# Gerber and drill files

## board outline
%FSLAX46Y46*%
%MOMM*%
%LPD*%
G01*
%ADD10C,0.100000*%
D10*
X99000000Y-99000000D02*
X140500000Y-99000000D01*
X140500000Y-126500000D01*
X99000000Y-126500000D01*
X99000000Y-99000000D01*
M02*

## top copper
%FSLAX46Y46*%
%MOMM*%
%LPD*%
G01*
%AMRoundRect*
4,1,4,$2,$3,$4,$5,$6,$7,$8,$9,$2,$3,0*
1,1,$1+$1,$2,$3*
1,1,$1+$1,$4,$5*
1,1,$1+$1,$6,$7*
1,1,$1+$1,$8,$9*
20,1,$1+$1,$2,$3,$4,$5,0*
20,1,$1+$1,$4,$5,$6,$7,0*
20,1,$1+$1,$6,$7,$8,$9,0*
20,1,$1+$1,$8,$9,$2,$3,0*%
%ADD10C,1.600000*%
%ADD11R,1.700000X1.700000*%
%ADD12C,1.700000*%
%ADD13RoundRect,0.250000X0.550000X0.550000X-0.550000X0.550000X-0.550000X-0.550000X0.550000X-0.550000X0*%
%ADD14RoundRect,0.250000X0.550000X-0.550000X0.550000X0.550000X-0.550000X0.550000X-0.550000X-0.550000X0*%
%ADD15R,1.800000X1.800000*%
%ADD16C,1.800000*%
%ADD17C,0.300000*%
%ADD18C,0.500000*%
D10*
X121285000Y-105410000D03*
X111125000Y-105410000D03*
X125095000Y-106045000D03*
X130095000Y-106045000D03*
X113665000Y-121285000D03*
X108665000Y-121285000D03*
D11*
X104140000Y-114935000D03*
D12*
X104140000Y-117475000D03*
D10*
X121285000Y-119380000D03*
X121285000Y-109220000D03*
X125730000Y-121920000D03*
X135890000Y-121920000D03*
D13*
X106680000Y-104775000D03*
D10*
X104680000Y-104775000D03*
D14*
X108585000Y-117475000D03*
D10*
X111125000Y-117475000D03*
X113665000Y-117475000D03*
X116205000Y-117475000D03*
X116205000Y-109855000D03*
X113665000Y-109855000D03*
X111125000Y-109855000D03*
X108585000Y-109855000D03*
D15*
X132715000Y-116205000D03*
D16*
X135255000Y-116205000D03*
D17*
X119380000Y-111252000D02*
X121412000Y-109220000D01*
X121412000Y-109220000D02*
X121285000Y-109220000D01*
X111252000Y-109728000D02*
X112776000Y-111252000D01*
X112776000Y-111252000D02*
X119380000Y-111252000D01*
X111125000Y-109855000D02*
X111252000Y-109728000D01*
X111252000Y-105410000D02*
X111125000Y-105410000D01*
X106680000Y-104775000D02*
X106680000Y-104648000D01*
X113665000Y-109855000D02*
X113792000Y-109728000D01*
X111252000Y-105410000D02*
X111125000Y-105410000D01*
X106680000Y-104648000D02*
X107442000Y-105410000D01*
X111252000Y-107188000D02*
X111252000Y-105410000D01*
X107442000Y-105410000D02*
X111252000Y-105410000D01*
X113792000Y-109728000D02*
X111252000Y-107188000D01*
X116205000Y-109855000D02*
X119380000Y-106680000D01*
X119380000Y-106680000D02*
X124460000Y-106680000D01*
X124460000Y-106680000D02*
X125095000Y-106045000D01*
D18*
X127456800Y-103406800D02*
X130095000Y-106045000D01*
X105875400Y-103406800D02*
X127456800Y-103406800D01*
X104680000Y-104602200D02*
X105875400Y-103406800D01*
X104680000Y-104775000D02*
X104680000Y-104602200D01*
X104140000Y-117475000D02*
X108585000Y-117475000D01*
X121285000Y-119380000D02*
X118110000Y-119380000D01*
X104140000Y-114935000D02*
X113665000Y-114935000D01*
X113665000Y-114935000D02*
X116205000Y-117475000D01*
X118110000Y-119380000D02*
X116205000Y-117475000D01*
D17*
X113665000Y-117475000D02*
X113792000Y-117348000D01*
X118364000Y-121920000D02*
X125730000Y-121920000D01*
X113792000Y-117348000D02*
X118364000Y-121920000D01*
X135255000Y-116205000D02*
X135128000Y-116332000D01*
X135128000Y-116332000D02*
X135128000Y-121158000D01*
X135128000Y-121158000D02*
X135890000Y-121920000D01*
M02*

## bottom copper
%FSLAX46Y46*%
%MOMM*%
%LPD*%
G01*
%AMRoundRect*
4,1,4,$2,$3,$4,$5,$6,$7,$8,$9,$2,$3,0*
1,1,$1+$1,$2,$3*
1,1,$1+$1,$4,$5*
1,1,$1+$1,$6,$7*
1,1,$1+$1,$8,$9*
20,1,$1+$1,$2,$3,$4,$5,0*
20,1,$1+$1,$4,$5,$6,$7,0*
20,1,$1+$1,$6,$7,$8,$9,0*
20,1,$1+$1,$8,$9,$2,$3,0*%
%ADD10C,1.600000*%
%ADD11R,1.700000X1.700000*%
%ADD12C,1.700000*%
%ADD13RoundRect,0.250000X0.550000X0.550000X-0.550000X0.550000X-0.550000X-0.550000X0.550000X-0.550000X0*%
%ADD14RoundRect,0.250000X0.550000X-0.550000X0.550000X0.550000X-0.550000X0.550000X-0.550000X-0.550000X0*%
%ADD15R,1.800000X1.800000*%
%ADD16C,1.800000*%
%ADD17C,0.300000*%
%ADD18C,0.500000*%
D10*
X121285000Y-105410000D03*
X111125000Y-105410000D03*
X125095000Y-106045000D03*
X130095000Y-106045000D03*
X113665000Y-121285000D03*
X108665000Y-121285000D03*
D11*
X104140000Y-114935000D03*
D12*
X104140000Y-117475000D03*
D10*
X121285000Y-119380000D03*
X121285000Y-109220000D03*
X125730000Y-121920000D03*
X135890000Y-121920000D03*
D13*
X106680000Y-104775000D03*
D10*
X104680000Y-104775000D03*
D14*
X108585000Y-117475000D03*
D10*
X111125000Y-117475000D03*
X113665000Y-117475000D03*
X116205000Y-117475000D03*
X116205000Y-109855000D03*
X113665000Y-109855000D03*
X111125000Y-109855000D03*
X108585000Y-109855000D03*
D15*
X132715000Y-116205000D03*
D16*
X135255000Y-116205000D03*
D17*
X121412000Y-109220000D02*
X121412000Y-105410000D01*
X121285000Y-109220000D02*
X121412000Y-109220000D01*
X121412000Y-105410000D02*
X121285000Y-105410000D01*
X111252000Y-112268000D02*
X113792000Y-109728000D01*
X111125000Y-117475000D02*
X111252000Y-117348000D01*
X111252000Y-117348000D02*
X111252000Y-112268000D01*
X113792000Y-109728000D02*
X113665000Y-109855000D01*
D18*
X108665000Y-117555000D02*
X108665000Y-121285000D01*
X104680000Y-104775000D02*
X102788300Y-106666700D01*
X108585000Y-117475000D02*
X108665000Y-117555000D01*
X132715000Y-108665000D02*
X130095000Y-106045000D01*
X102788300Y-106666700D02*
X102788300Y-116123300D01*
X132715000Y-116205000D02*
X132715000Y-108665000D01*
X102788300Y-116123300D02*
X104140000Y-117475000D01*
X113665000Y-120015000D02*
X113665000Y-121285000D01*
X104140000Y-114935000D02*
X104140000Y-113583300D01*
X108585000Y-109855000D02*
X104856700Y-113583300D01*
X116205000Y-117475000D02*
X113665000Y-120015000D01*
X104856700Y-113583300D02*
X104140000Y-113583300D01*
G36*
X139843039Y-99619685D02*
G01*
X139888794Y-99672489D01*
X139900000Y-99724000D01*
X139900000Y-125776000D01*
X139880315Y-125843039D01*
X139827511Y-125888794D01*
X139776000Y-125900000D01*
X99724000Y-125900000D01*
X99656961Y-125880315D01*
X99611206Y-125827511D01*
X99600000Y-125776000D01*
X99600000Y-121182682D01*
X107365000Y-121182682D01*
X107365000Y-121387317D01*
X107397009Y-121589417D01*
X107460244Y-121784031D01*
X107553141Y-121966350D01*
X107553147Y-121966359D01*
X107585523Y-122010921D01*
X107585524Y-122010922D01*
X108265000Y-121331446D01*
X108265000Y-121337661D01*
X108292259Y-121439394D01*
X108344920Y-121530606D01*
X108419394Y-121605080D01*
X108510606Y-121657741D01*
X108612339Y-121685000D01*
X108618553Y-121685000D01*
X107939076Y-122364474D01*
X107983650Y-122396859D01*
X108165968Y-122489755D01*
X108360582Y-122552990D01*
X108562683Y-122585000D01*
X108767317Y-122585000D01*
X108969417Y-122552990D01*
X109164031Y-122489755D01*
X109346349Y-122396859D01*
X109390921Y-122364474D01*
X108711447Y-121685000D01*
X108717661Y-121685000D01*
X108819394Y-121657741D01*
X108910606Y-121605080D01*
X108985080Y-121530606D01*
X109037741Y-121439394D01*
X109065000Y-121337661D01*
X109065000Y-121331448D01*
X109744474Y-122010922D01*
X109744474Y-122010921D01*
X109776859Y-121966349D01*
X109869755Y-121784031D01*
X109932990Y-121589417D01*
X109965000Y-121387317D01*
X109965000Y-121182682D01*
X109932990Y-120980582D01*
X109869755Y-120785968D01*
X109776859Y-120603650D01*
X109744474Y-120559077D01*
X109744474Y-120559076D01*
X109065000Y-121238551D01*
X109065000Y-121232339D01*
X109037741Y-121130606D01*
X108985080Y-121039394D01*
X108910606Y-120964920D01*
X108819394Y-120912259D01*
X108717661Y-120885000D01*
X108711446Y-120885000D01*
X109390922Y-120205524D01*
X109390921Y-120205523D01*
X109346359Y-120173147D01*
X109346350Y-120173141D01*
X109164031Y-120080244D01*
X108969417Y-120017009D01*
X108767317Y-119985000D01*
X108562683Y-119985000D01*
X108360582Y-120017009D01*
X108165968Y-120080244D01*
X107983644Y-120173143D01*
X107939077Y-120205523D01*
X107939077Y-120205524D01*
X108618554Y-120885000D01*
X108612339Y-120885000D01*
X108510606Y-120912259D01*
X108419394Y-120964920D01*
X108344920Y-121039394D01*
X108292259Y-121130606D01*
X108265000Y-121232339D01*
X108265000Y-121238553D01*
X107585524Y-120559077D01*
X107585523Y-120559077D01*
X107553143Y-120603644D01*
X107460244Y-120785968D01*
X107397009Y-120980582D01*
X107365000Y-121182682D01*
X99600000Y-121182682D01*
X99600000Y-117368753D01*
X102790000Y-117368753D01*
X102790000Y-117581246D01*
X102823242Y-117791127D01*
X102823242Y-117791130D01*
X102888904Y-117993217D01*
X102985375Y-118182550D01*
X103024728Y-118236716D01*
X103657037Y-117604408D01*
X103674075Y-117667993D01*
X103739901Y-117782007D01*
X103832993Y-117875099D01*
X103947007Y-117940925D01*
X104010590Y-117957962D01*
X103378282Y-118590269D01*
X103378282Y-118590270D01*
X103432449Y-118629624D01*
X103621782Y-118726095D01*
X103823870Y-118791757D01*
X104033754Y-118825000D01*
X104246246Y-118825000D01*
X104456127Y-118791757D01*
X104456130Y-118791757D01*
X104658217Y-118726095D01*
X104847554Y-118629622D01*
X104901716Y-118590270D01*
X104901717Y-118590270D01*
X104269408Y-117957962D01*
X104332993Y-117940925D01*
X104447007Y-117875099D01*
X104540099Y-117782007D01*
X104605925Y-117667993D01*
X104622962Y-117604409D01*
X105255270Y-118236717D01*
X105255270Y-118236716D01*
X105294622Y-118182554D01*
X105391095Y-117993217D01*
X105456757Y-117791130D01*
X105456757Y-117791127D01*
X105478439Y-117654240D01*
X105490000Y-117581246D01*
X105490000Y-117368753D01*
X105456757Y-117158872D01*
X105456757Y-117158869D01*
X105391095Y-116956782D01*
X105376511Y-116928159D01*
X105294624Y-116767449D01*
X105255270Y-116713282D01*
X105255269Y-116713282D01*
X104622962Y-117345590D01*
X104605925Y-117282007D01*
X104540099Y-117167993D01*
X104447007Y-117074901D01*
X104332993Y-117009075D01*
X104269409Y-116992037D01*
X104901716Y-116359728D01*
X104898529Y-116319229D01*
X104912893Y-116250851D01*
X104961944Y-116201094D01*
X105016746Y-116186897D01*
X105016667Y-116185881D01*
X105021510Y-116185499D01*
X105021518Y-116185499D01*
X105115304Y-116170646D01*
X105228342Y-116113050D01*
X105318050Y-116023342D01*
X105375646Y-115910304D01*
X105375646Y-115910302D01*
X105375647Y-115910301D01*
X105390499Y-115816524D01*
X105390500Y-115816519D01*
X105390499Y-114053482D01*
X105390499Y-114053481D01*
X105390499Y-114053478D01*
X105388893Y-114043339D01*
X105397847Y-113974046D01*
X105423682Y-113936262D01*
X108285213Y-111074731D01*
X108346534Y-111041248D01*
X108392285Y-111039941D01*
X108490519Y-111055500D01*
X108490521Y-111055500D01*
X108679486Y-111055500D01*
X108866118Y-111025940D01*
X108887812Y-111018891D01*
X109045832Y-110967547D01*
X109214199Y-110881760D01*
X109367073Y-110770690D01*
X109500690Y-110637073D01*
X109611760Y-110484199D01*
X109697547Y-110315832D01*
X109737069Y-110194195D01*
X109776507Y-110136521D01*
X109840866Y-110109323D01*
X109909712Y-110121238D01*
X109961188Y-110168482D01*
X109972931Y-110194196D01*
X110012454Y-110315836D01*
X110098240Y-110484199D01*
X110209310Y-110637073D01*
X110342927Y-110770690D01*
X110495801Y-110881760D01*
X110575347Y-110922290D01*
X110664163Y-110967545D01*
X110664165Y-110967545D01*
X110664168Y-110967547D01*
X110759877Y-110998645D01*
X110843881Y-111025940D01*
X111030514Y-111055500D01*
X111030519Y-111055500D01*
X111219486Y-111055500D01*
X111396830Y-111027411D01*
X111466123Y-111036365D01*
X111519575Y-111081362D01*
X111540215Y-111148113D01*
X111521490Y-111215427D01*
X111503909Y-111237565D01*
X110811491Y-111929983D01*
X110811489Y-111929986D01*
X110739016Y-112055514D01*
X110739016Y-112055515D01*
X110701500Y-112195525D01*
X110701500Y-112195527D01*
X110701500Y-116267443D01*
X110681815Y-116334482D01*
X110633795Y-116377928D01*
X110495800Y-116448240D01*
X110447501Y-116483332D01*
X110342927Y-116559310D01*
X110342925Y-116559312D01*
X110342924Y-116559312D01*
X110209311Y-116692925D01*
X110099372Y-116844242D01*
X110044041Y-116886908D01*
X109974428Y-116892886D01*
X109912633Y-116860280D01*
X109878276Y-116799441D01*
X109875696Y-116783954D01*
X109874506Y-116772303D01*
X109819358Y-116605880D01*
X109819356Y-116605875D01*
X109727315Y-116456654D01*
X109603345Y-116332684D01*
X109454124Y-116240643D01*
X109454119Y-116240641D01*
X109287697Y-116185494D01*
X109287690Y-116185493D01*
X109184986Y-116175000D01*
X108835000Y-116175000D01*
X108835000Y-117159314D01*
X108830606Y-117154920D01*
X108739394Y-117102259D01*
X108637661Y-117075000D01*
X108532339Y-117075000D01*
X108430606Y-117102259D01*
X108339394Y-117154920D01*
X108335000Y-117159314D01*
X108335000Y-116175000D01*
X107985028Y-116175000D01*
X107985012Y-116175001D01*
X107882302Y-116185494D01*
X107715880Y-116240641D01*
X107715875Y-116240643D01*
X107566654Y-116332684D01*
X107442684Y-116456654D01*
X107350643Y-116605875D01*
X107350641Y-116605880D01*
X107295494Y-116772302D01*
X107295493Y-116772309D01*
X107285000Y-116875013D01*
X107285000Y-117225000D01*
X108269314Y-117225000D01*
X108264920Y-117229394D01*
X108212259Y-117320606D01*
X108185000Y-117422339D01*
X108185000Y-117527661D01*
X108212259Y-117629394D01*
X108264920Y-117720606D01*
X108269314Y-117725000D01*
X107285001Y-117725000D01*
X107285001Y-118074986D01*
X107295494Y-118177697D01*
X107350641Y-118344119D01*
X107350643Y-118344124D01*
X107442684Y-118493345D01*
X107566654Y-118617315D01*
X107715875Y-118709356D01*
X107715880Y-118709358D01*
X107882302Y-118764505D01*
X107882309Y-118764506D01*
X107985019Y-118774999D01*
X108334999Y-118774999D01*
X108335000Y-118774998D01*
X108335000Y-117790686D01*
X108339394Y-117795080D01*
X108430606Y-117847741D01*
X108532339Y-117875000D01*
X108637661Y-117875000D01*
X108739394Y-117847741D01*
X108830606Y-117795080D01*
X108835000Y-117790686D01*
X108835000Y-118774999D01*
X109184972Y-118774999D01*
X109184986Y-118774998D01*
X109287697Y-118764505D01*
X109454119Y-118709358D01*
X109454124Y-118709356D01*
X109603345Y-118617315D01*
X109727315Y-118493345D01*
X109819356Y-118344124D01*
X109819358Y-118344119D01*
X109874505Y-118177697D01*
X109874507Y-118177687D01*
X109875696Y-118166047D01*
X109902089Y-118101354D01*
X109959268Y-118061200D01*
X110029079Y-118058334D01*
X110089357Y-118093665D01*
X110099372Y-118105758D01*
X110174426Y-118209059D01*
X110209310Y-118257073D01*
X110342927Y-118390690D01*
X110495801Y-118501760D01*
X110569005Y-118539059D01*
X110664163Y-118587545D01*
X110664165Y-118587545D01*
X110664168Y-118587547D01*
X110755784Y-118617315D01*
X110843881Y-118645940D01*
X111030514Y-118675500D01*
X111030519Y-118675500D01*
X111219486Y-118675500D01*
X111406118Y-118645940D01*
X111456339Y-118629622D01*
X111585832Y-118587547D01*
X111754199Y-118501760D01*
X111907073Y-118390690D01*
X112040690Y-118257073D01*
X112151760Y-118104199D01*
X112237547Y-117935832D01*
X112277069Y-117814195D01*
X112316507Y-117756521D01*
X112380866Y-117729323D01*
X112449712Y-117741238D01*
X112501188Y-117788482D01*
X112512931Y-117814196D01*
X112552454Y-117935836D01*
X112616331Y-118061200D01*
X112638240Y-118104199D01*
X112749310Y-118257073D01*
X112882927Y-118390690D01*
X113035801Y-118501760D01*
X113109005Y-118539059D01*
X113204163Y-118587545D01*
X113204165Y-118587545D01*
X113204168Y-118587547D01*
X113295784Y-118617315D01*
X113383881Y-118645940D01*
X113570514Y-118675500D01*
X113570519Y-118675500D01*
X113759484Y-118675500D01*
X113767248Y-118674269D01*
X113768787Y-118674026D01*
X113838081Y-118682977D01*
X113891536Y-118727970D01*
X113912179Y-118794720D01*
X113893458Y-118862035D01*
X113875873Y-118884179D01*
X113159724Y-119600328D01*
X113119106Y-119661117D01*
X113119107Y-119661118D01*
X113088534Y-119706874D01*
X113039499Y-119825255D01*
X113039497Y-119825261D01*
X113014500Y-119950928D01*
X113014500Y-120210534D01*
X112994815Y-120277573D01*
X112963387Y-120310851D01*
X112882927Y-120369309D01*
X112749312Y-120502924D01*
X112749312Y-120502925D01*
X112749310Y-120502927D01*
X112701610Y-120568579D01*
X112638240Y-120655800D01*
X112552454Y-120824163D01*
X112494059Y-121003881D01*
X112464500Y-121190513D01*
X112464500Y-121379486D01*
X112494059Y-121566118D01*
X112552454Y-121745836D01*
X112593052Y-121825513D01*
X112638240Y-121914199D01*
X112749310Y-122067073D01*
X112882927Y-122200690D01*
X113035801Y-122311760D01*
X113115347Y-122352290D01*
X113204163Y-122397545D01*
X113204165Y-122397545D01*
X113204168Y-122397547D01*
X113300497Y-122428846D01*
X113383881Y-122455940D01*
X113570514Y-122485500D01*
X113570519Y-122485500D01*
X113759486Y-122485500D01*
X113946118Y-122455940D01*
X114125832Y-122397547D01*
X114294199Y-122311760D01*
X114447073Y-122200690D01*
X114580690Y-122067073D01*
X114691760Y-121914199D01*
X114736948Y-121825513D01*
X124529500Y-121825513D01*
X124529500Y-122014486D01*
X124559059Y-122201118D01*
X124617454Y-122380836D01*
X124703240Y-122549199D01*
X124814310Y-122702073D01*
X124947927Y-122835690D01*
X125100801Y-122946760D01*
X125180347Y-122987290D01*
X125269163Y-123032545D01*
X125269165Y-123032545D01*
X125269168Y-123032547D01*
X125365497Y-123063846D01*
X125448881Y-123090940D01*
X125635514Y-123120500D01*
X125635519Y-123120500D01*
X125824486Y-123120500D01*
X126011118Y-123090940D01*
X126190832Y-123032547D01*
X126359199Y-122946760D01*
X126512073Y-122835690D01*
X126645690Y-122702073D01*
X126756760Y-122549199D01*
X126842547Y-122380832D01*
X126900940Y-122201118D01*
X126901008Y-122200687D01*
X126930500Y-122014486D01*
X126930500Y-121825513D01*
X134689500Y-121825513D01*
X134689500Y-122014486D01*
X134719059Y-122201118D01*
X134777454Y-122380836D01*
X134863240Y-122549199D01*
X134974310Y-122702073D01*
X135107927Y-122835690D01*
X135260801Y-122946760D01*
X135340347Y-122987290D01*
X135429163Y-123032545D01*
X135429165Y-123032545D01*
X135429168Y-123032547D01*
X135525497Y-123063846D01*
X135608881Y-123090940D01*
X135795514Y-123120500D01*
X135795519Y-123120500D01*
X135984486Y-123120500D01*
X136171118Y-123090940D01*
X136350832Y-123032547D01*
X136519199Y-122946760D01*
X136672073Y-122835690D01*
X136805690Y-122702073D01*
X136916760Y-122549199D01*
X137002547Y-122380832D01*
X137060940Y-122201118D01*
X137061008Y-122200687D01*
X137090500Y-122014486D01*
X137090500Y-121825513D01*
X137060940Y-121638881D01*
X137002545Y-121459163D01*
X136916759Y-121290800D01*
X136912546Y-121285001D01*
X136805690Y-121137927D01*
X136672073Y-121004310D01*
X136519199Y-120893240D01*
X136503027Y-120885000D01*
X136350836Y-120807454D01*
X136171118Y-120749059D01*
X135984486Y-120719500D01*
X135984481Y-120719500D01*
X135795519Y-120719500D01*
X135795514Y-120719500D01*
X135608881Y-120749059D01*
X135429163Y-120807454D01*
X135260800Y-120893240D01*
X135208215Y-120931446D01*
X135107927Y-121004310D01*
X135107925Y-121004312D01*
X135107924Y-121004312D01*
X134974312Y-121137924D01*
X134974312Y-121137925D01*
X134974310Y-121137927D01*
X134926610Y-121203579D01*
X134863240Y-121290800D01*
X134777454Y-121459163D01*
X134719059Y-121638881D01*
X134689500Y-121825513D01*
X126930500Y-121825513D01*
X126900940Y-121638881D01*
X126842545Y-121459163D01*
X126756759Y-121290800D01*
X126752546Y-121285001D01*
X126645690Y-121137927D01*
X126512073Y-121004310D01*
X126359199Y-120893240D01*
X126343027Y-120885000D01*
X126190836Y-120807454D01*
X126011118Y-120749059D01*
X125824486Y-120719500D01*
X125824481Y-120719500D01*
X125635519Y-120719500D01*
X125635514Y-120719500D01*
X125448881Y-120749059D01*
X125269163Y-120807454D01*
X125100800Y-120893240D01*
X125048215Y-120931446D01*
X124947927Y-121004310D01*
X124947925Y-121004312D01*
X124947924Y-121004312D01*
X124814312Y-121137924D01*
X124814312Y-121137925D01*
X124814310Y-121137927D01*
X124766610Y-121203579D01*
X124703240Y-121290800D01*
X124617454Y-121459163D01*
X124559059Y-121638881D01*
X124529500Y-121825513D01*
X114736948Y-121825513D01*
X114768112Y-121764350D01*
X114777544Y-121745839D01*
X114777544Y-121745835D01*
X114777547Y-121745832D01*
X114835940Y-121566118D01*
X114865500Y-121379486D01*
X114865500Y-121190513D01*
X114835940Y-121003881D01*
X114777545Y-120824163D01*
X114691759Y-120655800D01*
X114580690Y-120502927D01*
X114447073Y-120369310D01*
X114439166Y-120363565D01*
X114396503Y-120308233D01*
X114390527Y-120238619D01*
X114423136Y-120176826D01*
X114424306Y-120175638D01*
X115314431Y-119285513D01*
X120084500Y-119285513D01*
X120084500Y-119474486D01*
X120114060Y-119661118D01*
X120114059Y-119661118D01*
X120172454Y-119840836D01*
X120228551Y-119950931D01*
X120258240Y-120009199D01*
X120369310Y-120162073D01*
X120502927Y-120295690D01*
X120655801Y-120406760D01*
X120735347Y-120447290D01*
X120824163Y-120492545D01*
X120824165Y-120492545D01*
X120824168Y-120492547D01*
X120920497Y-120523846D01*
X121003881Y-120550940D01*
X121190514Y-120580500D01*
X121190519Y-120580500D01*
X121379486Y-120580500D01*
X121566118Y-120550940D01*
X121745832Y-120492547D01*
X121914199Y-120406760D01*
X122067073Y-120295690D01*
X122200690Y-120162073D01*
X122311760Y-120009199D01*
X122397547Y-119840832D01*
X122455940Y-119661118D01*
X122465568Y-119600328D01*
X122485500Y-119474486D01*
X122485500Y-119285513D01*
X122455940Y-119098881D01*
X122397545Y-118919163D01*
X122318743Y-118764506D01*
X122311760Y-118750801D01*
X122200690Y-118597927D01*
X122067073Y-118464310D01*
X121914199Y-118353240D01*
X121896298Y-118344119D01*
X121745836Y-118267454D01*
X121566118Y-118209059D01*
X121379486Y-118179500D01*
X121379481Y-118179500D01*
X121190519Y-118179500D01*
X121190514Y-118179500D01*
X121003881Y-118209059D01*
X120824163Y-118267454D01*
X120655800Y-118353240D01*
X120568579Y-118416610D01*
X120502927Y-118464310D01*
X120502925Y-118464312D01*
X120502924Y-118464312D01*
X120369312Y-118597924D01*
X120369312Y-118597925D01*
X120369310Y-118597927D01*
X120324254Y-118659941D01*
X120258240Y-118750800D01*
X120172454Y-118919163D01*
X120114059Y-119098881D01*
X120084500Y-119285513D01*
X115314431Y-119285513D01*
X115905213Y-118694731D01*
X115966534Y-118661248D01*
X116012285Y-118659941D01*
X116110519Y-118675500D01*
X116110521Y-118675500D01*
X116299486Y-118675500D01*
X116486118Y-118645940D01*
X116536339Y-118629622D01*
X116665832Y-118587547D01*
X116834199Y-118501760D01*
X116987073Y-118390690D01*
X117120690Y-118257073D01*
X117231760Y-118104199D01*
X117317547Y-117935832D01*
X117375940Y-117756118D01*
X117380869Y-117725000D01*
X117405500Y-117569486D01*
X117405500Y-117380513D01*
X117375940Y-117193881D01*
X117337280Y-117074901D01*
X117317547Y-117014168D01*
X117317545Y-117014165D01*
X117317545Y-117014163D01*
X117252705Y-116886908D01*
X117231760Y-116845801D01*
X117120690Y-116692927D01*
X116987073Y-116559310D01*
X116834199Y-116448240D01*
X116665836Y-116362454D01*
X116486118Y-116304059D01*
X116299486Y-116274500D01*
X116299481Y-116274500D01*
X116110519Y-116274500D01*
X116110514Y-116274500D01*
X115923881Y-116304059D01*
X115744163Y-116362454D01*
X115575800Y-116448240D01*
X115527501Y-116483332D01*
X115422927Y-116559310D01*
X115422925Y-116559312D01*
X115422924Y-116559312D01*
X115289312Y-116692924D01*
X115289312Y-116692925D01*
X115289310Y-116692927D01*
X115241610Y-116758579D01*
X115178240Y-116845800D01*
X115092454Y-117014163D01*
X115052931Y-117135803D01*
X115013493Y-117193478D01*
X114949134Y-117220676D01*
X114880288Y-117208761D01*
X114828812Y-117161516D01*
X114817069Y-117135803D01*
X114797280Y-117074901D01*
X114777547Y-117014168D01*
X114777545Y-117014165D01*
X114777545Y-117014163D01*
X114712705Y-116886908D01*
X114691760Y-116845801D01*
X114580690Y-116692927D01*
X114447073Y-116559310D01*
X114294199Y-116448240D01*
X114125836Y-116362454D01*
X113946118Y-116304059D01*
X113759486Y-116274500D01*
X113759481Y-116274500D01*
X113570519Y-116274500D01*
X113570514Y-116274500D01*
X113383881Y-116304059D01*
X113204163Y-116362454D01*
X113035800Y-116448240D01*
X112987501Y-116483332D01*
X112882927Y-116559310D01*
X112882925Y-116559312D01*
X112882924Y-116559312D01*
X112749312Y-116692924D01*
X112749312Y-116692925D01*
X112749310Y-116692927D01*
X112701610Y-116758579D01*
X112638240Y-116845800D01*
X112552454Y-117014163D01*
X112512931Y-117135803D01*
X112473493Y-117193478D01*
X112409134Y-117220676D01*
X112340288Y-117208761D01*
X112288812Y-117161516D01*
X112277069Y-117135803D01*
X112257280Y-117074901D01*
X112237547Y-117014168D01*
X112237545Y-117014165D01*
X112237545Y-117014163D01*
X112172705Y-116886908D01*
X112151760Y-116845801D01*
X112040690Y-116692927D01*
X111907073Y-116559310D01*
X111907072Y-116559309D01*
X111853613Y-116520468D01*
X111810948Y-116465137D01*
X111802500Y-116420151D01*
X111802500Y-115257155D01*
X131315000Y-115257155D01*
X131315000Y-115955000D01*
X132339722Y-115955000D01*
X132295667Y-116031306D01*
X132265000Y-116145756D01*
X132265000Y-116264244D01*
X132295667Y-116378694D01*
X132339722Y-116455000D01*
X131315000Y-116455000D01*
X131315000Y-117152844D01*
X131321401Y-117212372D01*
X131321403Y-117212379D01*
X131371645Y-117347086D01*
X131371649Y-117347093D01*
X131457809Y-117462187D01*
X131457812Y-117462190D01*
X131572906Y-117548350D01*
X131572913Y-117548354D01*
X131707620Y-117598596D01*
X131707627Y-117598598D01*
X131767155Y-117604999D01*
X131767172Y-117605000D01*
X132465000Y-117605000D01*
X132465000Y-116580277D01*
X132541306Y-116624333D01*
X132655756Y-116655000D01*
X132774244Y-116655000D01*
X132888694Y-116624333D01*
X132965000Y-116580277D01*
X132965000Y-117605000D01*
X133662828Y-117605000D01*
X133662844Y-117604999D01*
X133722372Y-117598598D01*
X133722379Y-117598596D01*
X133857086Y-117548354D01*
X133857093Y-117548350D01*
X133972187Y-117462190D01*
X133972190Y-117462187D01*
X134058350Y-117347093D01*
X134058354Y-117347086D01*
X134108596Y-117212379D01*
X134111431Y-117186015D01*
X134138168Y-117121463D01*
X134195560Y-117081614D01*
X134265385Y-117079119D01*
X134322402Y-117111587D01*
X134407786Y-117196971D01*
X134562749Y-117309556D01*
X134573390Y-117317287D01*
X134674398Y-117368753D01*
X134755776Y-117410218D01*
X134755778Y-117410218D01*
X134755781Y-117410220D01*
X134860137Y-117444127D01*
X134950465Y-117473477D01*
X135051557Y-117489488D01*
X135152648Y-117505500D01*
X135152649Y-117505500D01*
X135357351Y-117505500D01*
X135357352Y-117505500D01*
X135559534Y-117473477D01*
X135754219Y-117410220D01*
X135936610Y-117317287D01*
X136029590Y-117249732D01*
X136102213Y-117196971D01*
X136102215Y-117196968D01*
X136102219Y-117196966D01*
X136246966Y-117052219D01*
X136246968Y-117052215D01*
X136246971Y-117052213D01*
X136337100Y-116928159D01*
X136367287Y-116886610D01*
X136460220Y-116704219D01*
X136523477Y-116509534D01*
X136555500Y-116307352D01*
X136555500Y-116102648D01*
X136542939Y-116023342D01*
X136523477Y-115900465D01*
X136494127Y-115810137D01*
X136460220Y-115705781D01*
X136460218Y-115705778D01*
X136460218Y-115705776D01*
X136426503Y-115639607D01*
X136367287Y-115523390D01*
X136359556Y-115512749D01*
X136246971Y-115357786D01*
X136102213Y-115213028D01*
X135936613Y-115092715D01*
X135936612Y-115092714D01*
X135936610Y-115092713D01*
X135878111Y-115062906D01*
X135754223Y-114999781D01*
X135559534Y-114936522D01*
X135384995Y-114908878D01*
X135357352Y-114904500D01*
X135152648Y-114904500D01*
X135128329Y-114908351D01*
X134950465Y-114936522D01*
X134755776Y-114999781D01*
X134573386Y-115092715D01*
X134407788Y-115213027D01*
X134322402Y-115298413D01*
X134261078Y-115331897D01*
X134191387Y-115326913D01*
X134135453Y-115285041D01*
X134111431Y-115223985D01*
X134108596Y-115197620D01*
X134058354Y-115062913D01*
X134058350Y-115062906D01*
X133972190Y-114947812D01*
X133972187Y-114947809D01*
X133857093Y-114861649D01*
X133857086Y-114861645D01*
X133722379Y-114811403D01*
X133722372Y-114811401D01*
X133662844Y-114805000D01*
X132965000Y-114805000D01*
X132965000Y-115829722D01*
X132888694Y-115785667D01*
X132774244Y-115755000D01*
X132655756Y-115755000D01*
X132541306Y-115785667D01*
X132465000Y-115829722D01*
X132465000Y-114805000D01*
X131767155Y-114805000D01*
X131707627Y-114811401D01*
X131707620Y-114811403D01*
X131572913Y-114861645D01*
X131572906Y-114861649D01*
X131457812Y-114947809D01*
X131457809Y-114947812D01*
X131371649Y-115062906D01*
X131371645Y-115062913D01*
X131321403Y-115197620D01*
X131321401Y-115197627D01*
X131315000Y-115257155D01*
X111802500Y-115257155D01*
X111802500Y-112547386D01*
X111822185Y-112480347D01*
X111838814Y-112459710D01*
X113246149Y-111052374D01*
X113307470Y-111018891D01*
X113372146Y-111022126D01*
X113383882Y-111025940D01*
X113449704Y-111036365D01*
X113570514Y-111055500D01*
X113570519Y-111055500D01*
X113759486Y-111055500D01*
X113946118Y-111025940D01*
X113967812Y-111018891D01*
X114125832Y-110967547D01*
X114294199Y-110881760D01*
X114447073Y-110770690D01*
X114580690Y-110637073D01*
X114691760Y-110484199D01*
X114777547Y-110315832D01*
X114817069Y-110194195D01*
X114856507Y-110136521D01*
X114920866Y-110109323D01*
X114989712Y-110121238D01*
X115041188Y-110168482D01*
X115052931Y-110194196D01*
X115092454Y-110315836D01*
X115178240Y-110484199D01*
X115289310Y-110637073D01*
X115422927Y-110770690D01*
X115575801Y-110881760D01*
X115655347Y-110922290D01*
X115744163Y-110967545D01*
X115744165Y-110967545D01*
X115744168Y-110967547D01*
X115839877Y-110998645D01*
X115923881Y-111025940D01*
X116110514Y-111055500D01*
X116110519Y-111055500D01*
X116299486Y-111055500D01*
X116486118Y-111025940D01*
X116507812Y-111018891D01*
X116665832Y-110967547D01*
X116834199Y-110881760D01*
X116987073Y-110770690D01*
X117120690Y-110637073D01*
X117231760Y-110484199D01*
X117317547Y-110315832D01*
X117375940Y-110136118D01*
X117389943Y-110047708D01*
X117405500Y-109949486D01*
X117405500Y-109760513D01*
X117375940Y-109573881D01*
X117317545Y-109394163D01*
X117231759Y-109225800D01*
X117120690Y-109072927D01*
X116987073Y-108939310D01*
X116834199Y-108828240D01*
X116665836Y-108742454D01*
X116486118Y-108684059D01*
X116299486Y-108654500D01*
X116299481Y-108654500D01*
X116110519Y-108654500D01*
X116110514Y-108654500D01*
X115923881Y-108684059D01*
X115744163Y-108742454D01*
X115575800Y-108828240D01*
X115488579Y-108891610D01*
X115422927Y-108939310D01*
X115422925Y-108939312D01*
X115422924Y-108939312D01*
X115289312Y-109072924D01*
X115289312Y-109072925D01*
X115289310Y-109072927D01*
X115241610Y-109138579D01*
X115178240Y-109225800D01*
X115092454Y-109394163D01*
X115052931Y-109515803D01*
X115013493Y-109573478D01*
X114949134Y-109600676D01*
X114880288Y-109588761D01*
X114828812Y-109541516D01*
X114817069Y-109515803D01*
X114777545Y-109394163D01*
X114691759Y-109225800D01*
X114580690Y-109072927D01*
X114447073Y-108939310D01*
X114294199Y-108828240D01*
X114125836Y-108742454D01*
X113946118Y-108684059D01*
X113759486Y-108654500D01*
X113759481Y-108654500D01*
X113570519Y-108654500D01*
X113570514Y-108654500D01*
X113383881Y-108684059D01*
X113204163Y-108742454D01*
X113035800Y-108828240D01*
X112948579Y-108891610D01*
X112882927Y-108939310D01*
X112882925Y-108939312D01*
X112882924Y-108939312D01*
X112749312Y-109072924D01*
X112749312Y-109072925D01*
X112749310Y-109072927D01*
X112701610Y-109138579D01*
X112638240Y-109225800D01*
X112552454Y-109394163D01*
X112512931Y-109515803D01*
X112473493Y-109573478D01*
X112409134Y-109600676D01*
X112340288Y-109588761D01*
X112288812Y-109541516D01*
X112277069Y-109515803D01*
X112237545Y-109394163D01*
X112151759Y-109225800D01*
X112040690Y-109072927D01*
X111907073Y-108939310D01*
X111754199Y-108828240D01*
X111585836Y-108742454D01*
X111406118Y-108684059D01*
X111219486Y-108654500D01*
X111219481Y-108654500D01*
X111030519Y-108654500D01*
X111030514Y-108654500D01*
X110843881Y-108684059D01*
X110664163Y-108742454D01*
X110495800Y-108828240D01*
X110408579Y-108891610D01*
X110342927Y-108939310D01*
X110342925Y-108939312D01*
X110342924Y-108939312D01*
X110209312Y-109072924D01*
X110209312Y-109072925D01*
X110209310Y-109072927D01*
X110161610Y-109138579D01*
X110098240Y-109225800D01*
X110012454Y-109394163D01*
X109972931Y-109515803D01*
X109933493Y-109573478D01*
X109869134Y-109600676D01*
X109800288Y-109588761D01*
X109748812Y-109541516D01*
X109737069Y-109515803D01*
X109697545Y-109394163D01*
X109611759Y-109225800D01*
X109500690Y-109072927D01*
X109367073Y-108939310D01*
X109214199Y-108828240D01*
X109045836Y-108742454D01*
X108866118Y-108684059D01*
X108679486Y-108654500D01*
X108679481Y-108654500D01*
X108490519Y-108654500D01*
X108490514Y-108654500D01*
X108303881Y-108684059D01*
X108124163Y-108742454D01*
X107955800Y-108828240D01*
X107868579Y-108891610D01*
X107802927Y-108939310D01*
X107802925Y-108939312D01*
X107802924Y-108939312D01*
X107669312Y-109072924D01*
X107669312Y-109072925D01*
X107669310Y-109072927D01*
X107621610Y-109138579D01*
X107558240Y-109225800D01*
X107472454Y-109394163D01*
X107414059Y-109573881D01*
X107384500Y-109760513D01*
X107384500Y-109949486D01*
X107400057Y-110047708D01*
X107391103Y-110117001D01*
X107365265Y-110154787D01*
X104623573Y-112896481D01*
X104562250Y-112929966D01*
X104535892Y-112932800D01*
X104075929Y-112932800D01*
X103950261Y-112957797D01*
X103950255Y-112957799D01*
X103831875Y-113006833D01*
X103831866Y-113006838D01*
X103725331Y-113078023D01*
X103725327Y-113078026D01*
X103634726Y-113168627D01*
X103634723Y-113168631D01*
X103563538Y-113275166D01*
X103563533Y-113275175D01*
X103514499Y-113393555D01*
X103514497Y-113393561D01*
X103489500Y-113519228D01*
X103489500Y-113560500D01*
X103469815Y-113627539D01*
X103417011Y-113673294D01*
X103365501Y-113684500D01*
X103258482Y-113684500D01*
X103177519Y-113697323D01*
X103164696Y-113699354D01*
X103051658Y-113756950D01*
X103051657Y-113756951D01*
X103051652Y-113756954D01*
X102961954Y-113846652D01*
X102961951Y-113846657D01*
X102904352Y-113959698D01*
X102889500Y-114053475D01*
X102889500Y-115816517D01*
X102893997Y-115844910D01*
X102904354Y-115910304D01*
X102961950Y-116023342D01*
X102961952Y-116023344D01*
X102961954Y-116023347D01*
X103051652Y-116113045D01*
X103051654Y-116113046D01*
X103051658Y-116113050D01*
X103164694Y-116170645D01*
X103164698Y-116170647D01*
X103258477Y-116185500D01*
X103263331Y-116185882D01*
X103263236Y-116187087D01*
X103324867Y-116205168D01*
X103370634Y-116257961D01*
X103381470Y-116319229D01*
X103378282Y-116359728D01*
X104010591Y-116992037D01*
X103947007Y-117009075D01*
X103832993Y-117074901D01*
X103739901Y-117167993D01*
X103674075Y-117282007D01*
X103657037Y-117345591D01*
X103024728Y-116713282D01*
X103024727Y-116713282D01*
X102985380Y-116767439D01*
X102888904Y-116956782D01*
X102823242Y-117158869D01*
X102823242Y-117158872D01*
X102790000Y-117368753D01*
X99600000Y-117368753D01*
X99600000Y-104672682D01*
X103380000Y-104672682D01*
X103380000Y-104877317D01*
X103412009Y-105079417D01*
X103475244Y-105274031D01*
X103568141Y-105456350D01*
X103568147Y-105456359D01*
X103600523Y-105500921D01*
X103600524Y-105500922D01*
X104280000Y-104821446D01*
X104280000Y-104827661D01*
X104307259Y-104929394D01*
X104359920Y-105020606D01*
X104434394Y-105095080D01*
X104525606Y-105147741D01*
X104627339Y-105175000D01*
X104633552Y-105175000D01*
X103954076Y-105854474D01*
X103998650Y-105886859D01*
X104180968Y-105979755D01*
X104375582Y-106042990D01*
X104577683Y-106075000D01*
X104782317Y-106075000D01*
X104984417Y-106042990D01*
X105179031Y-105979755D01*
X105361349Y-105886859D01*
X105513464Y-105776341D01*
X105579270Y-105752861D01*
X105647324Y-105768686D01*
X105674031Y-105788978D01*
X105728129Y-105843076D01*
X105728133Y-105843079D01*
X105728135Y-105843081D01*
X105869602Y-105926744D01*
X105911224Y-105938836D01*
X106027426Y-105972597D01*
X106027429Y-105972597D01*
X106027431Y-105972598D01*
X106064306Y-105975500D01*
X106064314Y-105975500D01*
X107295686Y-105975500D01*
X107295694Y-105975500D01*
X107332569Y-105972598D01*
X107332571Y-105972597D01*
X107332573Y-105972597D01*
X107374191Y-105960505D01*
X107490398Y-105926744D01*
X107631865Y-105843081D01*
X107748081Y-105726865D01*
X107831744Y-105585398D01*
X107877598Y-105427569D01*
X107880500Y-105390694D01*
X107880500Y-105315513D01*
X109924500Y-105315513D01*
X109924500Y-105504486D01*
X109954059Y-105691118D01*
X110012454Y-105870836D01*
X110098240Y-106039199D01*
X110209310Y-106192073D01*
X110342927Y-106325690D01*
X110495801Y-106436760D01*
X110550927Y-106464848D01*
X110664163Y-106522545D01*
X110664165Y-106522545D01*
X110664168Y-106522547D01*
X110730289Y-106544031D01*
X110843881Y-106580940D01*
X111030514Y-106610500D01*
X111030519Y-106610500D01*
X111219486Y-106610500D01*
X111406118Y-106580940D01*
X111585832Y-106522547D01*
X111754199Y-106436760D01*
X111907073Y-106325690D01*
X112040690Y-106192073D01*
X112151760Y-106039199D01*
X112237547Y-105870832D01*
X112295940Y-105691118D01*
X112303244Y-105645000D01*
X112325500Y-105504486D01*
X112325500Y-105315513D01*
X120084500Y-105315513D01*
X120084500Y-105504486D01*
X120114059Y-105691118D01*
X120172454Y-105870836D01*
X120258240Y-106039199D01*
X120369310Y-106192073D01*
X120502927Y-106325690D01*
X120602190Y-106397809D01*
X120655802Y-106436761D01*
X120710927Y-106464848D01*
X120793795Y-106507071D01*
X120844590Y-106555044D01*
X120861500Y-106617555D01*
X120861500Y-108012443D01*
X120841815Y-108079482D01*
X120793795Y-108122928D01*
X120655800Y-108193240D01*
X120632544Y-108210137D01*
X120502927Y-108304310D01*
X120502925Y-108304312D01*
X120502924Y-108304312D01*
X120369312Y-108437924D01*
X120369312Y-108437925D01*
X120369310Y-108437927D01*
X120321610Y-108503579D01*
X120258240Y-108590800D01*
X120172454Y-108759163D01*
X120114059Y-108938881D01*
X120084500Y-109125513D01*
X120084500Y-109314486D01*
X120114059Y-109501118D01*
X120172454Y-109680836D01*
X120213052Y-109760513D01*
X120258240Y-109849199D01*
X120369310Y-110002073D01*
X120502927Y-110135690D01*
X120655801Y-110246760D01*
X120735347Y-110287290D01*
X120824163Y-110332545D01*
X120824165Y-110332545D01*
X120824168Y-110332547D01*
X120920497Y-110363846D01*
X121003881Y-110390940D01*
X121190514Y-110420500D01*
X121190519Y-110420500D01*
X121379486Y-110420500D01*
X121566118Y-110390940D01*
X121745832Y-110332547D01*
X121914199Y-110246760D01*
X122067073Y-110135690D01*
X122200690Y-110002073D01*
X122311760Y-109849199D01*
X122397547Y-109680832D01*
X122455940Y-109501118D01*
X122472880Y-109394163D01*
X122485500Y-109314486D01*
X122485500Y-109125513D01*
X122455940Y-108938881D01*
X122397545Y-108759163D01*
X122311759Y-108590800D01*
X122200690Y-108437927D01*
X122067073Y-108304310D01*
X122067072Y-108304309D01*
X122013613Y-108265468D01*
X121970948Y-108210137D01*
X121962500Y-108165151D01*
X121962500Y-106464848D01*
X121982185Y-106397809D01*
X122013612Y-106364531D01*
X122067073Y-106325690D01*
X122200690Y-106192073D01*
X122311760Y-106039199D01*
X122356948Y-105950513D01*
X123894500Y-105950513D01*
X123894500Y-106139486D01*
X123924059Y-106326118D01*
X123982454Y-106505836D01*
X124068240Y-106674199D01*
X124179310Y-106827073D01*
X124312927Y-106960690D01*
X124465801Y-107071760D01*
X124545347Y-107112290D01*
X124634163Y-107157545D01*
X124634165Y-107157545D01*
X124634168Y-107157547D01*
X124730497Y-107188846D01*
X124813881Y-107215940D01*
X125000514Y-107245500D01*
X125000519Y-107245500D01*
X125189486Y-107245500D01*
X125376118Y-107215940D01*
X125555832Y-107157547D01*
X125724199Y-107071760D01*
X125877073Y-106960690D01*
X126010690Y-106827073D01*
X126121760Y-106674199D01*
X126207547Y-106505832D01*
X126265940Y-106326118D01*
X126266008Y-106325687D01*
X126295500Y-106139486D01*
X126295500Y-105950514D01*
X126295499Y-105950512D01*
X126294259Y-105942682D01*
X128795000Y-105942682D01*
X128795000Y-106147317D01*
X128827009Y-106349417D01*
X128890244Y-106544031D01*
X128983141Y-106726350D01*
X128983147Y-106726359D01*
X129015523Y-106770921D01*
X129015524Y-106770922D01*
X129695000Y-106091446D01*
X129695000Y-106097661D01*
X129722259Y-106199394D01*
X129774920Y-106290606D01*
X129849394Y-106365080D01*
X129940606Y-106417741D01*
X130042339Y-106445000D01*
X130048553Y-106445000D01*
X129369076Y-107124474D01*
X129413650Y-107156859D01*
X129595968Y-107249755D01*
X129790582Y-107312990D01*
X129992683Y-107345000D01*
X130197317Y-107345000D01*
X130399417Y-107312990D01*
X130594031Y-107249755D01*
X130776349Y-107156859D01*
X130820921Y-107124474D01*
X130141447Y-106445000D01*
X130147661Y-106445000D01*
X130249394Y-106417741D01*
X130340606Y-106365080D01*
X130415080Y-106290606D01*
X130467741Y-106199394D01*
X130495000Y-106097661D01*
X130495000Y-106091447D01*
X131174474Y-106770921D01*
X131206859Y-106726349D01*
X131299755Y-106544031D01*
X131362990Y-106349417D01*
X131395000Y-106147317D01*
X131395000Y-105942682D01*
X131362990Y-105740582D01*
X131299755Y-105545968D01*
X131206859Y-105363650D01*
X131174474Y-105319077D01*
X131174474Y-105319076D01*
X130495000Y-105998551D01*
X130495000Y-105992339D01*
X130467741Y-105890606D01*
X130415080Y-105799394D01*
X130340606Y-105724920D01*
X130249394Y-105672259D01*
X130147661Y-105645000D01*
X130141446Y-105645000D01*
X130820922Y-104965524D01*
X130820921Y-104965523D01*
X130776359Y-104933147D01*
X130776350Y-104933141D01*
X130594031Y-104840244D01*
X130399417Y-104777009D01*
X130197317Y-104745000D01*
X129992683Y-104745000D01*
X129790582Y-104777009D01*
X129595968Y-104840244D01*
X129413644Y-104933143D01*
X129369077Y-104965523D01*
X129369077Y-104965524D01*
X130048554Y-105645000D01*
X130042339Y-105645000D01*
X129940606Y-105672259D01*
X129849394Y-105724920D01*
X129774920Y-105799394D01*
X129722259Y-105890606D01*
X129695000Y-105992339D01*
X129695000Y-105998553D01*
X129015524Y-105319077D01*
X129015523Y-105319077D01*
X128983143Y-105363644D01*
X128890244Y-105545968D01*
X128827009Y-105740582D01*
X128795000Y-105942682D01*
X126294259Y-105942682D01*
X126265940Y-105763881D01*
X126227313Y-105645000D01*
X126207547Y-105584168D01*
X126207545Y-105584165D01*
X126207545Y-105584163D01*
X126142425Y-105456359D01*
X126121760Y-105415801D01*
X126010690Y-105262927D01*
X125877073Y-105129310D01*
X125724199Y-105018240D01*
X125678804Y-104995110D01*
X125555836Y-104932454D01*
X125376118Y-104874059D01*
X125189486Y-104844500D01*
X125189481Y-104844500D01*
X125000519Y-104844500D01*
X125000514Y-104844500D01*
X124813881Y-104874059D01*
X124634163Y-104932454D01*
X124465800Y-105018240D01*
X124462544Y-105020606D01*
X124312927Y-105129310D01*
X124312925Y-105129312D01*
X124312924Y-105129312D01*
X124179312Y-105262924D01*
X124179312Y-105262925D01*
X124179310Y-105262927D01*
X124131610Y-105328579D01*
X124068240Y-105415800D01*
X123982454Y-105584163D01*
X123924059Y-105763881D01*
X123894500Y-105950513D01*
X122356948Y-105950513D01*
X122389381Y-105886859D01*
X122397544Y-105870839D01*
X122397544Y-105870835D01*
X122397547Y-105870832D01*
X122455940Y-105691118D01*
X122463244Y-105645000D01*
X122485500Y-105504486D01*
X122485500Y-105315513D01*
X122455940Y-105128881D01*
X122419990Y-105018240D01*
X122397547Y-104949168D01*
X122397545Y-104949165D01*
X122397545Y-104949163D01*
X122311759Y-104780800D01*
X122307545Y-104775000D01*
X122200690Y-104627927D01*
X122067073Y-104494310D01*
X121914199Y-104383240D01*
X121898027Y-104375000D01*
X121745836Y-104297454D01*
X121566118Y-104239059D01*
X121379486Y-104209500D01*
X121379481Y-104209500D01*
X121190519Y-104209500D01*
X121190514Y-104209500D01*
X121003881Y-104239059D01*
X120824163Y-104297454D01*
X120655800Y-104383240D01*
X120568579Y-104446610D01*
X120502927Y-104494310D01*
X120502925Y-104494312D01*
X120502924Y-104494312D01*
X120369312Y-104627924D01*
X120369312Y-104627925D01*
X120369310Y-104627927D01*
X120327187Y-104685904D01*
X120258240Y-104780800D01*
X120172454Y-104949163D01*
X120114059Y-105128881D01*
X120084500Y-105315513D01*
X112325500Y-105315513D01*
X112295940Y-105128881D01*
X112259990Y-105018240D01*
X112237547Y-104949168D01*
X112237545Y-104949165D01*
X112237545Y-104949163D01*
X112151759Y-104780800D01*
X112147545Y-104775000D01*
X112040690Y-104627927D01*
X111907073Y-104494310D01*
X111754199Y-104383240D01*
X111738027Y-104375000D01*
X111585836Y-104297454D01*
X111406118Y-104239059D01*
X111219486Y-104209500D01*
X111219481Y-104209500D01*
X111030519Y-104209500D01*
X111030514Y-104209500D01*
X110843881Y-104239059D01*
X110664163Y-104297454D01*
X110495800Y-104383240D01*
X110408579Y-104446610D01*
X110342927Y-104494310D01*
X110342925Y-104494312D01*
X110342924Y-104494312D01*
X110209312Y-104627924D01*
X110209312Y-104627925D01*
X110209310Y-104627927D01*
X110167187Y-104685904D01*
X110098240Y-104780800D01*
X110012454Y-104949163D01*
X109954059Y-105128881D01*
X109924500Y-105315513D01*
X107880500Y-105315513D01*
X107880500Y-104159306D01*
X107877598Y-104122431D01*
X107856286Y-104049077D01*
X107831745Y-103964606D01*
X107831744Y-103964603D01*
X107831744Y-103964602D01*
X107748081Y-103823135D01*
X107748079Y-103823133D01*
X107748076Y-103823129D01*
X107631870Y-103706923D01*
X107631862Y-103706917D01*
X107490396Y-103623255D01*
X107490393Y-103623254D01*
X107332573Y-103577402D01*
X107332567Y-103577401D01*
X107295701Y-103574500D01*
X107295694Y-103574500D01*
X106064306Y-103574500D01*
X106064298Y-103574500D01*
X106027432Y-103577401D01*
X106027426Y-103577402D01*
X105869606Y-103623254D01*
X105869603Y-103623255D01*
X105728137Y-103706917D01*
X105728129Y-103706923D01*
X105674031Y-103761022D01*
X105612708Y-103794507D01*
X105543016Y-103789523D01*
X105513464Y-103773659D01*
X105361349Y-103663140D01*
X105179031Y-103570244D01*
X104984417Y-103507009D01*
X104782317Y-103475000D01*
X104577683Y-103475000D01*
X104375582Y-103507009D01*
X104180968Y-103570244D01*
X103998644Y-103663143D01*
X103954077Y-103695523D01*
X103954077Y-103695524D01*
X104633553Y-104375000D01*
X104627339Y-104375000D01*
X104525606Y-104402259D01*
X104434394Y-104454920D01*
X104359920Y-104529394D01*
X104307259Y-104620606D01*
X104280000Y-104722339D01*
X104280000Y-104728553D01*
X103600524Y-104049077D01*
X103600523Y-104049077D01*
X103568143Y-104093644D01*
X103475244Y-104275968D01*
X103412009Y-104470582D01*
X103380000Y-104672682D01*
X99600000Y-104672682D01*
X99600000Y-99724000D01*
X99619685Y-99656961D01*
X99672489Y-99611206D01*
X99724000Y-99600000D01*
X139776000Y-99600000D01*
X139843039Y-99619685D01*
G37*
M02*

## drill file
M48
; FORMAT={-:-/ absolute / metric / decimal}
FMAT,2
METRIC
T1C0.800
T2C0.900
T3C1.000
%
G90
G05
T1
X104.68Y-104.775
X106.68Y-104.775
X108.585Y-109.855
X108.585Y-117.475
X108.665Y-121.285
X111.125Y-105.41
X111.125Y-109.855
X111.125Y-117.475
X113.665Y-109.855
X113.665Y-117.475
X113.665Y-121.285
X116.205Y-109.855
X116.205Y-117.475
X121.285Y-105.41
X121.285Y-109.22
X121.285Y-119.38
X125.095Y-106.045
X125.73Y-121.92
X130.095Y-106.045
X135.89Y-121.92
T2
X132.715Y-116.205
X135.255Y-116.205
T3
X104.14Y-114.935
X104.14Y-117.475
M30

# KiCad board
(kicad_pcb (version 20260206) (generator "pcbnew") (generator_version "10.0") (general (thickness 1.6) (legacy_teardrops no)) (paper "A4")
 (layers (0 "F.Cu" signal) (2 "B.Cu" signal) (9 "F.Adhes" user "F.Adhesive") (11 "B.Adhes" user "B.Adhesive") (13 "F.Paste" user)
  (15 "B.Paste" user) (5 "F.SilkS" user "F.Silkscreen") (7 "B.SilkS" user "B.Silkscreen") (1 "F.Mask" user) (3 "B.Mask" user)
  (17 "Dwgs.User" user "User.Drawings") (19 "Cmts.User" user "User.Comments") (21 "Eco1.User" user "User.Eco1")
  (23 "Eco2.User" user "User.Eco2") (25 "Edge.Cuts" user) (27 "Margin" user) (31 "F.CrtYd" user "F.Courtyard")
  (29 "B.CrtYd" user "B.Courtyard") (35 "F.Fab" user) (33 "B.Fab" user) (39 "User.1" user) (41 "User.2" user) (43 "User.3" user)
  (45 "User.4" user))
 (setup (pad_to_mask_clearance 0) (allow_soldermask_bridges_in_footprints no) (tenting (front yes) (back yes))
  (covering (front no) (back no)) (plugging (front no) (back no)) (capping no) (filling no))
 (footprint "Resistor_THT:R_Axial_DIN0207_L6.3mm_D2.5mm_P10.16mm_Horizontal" (layer "F.Cu") (at 121.285 105.41 180)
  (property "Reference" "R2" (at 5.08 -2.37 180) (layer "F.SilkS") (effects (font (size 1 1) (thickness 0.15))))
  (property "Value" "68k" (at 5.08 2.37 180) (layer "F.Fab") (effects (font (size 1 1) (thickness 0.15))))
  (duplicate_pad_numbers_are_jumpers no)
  (pad "1" thru_hole circle (at 0 0 180) (size 1.6 1.6) (drill 0.8) (layers "*.Cu" "*.Mask") (remove_unused_layers no)
   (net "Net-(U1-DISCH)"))
  (pad "2" thru_hole circle (at 10.16 0 180) (size 1.6 1.6) (drill 0.8) (layers "*.Cu" "*.Mask") (remove_unused_layers no)
   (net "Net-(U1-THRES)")))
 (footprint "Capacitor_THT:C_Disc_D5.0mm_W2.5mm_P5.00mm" (layer "F.Cu") (at 125.095 106.045)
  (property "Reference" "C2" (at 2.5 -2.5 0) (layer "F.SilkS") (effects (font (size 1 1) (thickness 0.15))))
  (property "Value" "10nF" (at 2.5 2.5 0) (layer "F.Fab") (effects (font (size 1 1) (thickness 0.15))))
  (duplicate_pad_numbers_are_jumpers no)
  (pad "1" thru_hole circle (at 0 0) (size 1.6 1.6) (drill 0.8) (layers "*.Cu" "*.Mask") (remove_unused_layers no) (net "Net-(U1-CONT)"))
  (pad "2" thru_hole circle (at 5 0) (size 1.6 1.6) (drill 0.8) (layers "*.Cu" "*.Mask") (remove_unused_layers no) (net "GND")))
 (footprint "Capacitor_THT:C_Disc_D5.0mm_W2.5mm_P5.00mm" (layer "F.Cu") (at 113.665 121.285 180)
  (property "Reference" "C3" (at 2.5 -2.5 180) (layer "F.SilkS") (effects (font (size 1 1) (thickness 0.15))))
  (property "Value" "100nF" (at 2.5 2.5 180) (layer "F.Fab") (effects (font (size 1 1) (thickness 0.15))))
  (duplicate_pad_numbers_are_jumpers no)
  (pad "1" thru_hole circle (at 0 0 180) (size 1.6 1.6) (drill 0.8) (layers "*.Cu" "*.Mask") (remove_unused_layers no) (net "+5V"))
  (pad "2" thru_hole circle (at 5 0 180) (size 1.6 1.6) (drill 0.8) (layers "*.Cu" "*.Mask") (remove_unused_layers no) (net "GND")))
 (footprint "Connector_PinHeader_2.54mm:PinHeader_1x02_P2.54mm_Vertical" (layer "F.Cu") (at 104.14 114.935)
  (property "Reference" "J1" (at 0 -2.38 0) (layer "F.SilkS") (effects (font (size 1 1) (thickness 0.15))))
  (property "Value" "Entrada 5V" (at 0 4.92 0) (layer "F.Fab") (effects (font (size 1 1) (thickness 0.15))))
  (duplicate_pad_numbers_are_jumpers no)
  (pad "1" thru_hole rect (at 0 0) (size 1.7 1.7) (drill 1) (layers "*.Cu" "*.Mask") (remove_unused_layers no) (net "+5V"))
  (pad "2" thru_hole circle (at 0 2.54) (size 1.7 1.7) (drill 1) (layers "*.Cu" "*.Mask") (remove_unused_layers no) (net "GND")))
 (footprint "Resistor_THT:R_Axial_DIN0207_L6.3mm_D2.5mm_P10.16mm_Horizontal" (layer "F.Cu") (at 121.285 119.38 90)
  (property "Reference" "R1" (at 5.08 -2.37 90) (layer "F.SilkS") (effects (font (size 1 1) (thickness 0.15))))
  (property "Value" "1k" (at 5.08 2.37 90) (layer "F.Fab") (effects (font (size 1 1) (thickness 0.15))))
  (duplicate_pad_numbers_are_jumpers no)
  (pad "1" thru_hole circle (at 0 0 90) (size 1.6 1.6) (drill 0.8) (layers "*.Cu" "*.Mask") (remove_unused_layers no) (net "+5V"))
  (pad "2" thru_hole circle (at 10.16 0 90) (size 1.6 1.6) (drill 0.8) (layers "*.Cu" "*.Mask") (remove_unused_layers no)
   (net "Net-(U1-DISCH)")))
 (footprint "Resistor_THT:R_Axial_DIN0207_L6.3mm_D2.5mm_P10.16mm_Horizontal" (layer "F.Cu") (at 125.73 121.92)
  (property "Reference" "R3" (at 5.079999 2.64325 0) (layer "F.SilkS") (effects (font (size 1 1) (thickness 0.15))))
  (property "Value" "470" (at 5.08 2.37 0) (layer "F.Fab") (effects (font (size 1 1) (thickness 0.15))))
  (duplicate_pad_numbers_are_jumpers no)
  (pad "1" thru_hole circle (at 0 0) (size 1.6 1.6) (drill 0.8) (layers "*.Cu" "*.Mask") (remove_unused_layers no) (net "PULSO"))
  (pad "2" thru_hole circle (at 10.16 0) (size 1.6 1.6) (drill 0.8) (layers "*.Cu" "*.Mask") (remove_unused_layers no) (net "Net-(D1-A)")))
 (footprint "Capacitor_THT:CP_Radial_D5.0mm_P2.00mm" (layer "F.Cu") (at 106.68 104.775 180)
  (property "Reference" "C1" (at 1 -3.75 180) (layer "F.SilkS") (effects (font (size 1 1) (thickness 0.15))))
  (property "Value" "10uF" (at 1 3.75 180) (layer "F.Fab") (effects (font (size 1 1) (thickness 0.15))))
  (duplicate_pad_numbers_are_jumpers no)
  (pad "1" thru_hole roundrect (at 0 0 180) (size 1.6 1.6) (drill 0.8) (layers "*.Cu" "*.Mask") (remove_unused_layers no)
   (roundrect_rratio 0.15625) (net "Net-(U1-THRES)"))
  (pad "2" thru_hole circle (at 2 0 180) (size 1.6 1.6) (drill 0.8) (layers "*.Cu" "*.Mask") (remove_unused_layers no) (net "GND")))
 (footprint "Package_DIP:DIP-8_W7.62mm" (layer "F.Cu") (at 108.585 117.475 90)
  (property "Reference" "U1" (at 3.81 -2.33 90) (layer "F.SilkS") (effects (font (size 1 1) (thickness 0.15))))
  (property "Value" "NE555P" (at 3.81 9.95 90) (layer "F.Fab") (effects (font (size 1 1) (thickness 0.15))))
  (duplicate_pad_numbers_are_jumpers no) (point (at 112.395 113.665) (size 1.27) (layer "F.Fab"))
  (pad "1" thru_hole roundrect (at 0 0 90) (size 1.6 1.6) (drill 0.8) (layers "*.Cu" "*.Mask") (remove_unused_layers no)
   (roundrect_rratio 0.15625) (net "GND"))
  (pad "2" thru_hole circle (at 0 2.54 90) (size 1.6 1.6) (drill 0.8) (layers "*.Cu" "*.Mask") (remove_unused_layers no)
   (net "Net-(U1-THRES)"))
  (pad "3" thru_hole circle (at 0 5.08 90) (size 1.6 1.6) (drill 0.8) (layers "*.Cu" "*.Mask") (remove_unused_layers no) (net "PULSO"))
  (pad "4" thru_hole circle (at 0 7.62 90) (size 1.6 1.6) (drill 0.8) (layers "*.Cu" "*.Mask") (remove_unused_layers no) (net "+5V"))
  (pad "5" thru_hole circle (at 7.62 7.62 90) (size 1.6 1.6) (drill 0.8) (layers "*.Cu" "*.Mask") (remove_unused_layers no)
   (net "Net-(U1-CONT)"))
  (pad "6" thru_hole circle (at 7.62 5.08 90) (size 1.6 1.6) (drill 0.8) (layers "*.Cu" "*.Mask") (remove_unused_layers no)
   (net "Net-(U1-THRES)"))
  (pad "7" thru_hole circle (at 7.62 2.54 90) (size 1.6 1.6) (drill 0.8) (layers "*.Cu" "*.Mask") (remove_unused_layers no)
   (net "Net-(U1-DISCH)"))
  (pad "8" thru_hole circle (at 7.62 0 90) (size 1.6 1.6) (drill 0.8) (layers "*.Cu" "*.Mask") (remove_unused_layers no) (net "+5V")))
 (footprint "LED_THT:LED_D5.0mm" (layer "F.Cu") (at 132.715 116.205)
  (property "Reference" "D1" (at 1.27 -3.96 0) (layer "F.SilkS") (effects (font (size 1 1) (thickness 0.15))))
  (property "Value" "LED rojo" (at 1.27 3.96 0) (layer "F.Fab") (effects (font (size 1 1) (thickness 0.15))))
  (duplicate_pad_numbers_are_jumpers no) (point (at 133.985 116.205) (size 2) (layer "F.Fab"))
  (pad "1" thru_hole rect (at 0 0) (size 1.8 1.8) (drill 0.9) (layers "*.Cu" "*.Mask") (remove_unused_layers no) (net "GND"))
  (pad "2" thru_hole circle (at 2.54 0) (size 1.8 1.8) (drill 0.9) (layers "*.Cu" "*.Mask") (remove_unused_layers no) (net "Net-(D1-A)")))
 (gr_rect (start 99 99) (end 140.5 126.5) (stroke (width 0.1) (type default)) (fill no) (layer "Edge.Cuts"))
 (segment (start 119.38 111.252) (end 121.412 109.22) (width 0.3) (layer "F.Cu") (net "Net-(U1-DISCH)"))
 (segment (start 121.412 109.22) (end 121.285 109.22) (width 0.3) (layer "F.Cu") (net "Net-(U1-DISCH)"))
 (segment (start 111.252 109.728) (end 112.776 111.252) (width 0.3) (layer "F.Cu") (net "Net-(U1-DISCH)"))
 (segment (start 112.776 111.252) (end 119.38 111.252) (width 0.3) (layer "F.Cu") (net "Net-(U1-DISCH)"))
 (segment (start 111.125 109.855) (end 111.252 109.728) (width 0.3) (layer "F.Cu") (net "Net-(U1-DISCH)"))
 (segment (start 121.412 109.22) (end 121.412 105.41) (width 0.3) (layer "B.Cu") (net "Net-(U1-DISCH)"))
 (segment (start 121.285 109.22) (end 121.412 109.22) (width 0.3) (layer "B.Cu") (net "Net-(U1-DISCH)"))
 (segment (start 121.412 105.41) (end 121.285 105.41) (width 0.3) (layer "B.Cu") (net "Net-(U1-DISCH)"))
 (segment (start 111.252 105.41) (end 111.125 105.41) (width 0.3) (layer "F.Cu") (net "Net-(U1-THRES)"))
 (segment (start 106.68 104.775) (end 106.68 104.648) (width 0.3) (layer "F.Cu") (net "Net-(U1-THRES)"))
 (segment (start 113.665 109.855) (end 113.792 109.728) (width 0.3) (layer "F.Cu") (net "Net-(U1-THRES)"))
 (segment (start 111.252 105.41) (end 111.125 105.41) (width 0.3) (layer "F.Cu") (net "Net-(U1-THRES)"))
 (segment (start 106.68 104.648) (end 107.442 105.41) (width 0.3) (layer "F.Cu") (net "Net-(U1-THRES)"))
 (segment (start 111.252 107.188) (end 111.252 105.41) (width 0.3) (layer "F.Cu") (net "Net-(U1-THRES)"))
 (segment (start 107.442 105.41) (end 111.252 105.41) (width 0.3) (layer "F.Cu") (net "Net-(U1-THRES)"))
 (segment (start 113.792 109.728) (end 111.252 107.188) (width 0.3) (layer "F.Cu") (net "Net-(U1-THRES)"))
 (segment (start 111.252 112.268) (end 113.792 109.728) (width 0.3) (layer "B.Cu") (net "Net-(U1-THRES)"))
 (segment (start 111.125 117.475) (end 111.252 117.348) (width 0.3) (layer "B.Cu") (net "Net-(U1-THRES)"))
 (segment (start 111.252 117.348) (end 111.252 112.268) (width 0.3) (layer "B.Cu") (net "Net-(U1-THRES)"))
 (segment (start 113.792 109.728) (end 113.665 109.855) (width 0.3) (layer "B.Cu") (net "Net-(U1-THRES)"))
 (segment (start 116.205 109.855) (end 119.38 106.68) (width 0.3) (layer "F.Cu") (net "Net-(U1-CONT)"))
 (segment (start 119.38 106.68) (end 124.46 106.68) (width 0.3) (layer "F.Cu") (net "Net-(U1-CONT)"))
 (segment (start 124.46 106.68) (end 125.095 106.045) (width 0.3) (layer "F.Cu") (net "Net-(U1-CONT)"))
 (segment (start 127.4568 103.4068) (end 130.095 106.045) (width 0.5) (layer "F.Cu") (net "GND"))
 (segment (start 105.8754 103.4068) (end 127.4568 103.4068) (width 0.5) (layer "F.Cu") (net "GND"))
 (segment (start 104.68 104.6022) (end 105.8754 103.4068) (width 0.5) (layer "F.Cu") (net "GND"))
 (segment (start 104.68 104.775) (end 104.68 104.6022) (width 0.5) (layer "F.Cu") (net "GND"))
 (segment (start 104.14 117.475) (end 108.585 117.475) (width 0.5) (layer "F.Cu") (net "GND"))
 (segment (start 108.665 117.555) (end 108.665 121.285) (width 0.5) (layer "B.Cu") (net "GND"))
 (segment (start 104.68 104.775) (end 102.7883 106.6667) (width 0.5) (layer "B.Cu") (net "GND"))
 (segment (start 108.585 117.475) (end 108.665 117.555) (width 0.5) (layer "B.Cu") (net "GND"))
 (segment (start 132.715 108.665) (end 130.095 106.045) (width 0.5) (layer "B.Cu") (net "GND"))
 (segment (start 102.7883 106.6667) (end 102.7883 116.1233) (width 0.5) (layer "B.Cu") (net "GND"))
 (segment (start 132.715 116.205) (end 132.715 108.665) (width 0.5) (layer "B.Cu") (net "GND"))
 (segment (start 102.7883 116.1233) (end 104.14 117.475) (width 0.5) (layer "B.Cu") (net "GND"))
 (segment (start 121.285 119.38) (end 118.11 119.38) (width 0.5) (layer "F.Cu") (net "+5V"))
 (segment (start 104.14 114.935) (end 113.665 114.935) (width 0.5) (layer "F.Cu") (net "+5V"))
 (segment (start 113.665 114.935) (end 116.205 117.475) (width 0.5) (layer "F.Cu") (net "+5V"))
 (segment (start 118.11 119.38) (end 116.205 117.475) (width 0.5) (layer "F.Cu") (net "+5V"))
 (segment (start 113.665 120.015) (end 113.665 121.285) (width 0.5) (layer "B.Cu") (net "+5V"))
 (segment (start 104.14 114.935) (end 104.14 113.5833) (width 0.5) (layer "B.Cu") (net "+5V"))
 (segment (start 108.585 109.855) (end 104.8567 113.5833) (width 0.5) (layer "B.Cu") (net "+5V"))
 (segment (start 116.205 117.475) (end 113.665 120.015) (width 0.5) (layer "B.Cu") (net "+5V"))
 (segment (start 104.8567 113.5833) (end 104.14 113.5833) (width 0.5) (layer "B.Cu") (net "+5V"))
 (segment (start 113.665 117.475) (end 113.792 117.348) (width 0.3) (layer "F.Cu") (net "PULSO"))
 (segment (start 118.364 121.92) (end 125.73 121.92) (width 0.3) (layer "F.Cu") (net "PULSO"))
 (segment (start 113.792 117.348) (end 118.364 121.92) (width 0.3) (layer "F.Cu") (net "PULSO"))
 (segment (start 135.255 116.205) (end 135.128 116.332) (width 0.3) (layer "F.Cu") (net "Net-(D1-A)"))
 (segment (start 135.128 116.332) (end 135.128 121.158) (width 0.3) (layer "F.Cu") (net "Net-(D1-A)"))
 (segment (start 135.128 121.158) (end 135.89 121.92) (width 0.3) (layer "F.Cu") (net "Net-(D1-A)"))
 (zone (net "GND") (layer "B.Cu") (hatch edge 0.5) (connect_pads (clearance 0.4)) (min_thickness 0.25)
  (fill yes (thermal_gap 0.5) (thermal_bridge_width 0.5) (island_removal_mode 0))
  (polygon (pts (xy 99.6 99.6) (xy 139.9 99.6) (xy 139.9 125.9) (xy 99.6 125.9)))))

